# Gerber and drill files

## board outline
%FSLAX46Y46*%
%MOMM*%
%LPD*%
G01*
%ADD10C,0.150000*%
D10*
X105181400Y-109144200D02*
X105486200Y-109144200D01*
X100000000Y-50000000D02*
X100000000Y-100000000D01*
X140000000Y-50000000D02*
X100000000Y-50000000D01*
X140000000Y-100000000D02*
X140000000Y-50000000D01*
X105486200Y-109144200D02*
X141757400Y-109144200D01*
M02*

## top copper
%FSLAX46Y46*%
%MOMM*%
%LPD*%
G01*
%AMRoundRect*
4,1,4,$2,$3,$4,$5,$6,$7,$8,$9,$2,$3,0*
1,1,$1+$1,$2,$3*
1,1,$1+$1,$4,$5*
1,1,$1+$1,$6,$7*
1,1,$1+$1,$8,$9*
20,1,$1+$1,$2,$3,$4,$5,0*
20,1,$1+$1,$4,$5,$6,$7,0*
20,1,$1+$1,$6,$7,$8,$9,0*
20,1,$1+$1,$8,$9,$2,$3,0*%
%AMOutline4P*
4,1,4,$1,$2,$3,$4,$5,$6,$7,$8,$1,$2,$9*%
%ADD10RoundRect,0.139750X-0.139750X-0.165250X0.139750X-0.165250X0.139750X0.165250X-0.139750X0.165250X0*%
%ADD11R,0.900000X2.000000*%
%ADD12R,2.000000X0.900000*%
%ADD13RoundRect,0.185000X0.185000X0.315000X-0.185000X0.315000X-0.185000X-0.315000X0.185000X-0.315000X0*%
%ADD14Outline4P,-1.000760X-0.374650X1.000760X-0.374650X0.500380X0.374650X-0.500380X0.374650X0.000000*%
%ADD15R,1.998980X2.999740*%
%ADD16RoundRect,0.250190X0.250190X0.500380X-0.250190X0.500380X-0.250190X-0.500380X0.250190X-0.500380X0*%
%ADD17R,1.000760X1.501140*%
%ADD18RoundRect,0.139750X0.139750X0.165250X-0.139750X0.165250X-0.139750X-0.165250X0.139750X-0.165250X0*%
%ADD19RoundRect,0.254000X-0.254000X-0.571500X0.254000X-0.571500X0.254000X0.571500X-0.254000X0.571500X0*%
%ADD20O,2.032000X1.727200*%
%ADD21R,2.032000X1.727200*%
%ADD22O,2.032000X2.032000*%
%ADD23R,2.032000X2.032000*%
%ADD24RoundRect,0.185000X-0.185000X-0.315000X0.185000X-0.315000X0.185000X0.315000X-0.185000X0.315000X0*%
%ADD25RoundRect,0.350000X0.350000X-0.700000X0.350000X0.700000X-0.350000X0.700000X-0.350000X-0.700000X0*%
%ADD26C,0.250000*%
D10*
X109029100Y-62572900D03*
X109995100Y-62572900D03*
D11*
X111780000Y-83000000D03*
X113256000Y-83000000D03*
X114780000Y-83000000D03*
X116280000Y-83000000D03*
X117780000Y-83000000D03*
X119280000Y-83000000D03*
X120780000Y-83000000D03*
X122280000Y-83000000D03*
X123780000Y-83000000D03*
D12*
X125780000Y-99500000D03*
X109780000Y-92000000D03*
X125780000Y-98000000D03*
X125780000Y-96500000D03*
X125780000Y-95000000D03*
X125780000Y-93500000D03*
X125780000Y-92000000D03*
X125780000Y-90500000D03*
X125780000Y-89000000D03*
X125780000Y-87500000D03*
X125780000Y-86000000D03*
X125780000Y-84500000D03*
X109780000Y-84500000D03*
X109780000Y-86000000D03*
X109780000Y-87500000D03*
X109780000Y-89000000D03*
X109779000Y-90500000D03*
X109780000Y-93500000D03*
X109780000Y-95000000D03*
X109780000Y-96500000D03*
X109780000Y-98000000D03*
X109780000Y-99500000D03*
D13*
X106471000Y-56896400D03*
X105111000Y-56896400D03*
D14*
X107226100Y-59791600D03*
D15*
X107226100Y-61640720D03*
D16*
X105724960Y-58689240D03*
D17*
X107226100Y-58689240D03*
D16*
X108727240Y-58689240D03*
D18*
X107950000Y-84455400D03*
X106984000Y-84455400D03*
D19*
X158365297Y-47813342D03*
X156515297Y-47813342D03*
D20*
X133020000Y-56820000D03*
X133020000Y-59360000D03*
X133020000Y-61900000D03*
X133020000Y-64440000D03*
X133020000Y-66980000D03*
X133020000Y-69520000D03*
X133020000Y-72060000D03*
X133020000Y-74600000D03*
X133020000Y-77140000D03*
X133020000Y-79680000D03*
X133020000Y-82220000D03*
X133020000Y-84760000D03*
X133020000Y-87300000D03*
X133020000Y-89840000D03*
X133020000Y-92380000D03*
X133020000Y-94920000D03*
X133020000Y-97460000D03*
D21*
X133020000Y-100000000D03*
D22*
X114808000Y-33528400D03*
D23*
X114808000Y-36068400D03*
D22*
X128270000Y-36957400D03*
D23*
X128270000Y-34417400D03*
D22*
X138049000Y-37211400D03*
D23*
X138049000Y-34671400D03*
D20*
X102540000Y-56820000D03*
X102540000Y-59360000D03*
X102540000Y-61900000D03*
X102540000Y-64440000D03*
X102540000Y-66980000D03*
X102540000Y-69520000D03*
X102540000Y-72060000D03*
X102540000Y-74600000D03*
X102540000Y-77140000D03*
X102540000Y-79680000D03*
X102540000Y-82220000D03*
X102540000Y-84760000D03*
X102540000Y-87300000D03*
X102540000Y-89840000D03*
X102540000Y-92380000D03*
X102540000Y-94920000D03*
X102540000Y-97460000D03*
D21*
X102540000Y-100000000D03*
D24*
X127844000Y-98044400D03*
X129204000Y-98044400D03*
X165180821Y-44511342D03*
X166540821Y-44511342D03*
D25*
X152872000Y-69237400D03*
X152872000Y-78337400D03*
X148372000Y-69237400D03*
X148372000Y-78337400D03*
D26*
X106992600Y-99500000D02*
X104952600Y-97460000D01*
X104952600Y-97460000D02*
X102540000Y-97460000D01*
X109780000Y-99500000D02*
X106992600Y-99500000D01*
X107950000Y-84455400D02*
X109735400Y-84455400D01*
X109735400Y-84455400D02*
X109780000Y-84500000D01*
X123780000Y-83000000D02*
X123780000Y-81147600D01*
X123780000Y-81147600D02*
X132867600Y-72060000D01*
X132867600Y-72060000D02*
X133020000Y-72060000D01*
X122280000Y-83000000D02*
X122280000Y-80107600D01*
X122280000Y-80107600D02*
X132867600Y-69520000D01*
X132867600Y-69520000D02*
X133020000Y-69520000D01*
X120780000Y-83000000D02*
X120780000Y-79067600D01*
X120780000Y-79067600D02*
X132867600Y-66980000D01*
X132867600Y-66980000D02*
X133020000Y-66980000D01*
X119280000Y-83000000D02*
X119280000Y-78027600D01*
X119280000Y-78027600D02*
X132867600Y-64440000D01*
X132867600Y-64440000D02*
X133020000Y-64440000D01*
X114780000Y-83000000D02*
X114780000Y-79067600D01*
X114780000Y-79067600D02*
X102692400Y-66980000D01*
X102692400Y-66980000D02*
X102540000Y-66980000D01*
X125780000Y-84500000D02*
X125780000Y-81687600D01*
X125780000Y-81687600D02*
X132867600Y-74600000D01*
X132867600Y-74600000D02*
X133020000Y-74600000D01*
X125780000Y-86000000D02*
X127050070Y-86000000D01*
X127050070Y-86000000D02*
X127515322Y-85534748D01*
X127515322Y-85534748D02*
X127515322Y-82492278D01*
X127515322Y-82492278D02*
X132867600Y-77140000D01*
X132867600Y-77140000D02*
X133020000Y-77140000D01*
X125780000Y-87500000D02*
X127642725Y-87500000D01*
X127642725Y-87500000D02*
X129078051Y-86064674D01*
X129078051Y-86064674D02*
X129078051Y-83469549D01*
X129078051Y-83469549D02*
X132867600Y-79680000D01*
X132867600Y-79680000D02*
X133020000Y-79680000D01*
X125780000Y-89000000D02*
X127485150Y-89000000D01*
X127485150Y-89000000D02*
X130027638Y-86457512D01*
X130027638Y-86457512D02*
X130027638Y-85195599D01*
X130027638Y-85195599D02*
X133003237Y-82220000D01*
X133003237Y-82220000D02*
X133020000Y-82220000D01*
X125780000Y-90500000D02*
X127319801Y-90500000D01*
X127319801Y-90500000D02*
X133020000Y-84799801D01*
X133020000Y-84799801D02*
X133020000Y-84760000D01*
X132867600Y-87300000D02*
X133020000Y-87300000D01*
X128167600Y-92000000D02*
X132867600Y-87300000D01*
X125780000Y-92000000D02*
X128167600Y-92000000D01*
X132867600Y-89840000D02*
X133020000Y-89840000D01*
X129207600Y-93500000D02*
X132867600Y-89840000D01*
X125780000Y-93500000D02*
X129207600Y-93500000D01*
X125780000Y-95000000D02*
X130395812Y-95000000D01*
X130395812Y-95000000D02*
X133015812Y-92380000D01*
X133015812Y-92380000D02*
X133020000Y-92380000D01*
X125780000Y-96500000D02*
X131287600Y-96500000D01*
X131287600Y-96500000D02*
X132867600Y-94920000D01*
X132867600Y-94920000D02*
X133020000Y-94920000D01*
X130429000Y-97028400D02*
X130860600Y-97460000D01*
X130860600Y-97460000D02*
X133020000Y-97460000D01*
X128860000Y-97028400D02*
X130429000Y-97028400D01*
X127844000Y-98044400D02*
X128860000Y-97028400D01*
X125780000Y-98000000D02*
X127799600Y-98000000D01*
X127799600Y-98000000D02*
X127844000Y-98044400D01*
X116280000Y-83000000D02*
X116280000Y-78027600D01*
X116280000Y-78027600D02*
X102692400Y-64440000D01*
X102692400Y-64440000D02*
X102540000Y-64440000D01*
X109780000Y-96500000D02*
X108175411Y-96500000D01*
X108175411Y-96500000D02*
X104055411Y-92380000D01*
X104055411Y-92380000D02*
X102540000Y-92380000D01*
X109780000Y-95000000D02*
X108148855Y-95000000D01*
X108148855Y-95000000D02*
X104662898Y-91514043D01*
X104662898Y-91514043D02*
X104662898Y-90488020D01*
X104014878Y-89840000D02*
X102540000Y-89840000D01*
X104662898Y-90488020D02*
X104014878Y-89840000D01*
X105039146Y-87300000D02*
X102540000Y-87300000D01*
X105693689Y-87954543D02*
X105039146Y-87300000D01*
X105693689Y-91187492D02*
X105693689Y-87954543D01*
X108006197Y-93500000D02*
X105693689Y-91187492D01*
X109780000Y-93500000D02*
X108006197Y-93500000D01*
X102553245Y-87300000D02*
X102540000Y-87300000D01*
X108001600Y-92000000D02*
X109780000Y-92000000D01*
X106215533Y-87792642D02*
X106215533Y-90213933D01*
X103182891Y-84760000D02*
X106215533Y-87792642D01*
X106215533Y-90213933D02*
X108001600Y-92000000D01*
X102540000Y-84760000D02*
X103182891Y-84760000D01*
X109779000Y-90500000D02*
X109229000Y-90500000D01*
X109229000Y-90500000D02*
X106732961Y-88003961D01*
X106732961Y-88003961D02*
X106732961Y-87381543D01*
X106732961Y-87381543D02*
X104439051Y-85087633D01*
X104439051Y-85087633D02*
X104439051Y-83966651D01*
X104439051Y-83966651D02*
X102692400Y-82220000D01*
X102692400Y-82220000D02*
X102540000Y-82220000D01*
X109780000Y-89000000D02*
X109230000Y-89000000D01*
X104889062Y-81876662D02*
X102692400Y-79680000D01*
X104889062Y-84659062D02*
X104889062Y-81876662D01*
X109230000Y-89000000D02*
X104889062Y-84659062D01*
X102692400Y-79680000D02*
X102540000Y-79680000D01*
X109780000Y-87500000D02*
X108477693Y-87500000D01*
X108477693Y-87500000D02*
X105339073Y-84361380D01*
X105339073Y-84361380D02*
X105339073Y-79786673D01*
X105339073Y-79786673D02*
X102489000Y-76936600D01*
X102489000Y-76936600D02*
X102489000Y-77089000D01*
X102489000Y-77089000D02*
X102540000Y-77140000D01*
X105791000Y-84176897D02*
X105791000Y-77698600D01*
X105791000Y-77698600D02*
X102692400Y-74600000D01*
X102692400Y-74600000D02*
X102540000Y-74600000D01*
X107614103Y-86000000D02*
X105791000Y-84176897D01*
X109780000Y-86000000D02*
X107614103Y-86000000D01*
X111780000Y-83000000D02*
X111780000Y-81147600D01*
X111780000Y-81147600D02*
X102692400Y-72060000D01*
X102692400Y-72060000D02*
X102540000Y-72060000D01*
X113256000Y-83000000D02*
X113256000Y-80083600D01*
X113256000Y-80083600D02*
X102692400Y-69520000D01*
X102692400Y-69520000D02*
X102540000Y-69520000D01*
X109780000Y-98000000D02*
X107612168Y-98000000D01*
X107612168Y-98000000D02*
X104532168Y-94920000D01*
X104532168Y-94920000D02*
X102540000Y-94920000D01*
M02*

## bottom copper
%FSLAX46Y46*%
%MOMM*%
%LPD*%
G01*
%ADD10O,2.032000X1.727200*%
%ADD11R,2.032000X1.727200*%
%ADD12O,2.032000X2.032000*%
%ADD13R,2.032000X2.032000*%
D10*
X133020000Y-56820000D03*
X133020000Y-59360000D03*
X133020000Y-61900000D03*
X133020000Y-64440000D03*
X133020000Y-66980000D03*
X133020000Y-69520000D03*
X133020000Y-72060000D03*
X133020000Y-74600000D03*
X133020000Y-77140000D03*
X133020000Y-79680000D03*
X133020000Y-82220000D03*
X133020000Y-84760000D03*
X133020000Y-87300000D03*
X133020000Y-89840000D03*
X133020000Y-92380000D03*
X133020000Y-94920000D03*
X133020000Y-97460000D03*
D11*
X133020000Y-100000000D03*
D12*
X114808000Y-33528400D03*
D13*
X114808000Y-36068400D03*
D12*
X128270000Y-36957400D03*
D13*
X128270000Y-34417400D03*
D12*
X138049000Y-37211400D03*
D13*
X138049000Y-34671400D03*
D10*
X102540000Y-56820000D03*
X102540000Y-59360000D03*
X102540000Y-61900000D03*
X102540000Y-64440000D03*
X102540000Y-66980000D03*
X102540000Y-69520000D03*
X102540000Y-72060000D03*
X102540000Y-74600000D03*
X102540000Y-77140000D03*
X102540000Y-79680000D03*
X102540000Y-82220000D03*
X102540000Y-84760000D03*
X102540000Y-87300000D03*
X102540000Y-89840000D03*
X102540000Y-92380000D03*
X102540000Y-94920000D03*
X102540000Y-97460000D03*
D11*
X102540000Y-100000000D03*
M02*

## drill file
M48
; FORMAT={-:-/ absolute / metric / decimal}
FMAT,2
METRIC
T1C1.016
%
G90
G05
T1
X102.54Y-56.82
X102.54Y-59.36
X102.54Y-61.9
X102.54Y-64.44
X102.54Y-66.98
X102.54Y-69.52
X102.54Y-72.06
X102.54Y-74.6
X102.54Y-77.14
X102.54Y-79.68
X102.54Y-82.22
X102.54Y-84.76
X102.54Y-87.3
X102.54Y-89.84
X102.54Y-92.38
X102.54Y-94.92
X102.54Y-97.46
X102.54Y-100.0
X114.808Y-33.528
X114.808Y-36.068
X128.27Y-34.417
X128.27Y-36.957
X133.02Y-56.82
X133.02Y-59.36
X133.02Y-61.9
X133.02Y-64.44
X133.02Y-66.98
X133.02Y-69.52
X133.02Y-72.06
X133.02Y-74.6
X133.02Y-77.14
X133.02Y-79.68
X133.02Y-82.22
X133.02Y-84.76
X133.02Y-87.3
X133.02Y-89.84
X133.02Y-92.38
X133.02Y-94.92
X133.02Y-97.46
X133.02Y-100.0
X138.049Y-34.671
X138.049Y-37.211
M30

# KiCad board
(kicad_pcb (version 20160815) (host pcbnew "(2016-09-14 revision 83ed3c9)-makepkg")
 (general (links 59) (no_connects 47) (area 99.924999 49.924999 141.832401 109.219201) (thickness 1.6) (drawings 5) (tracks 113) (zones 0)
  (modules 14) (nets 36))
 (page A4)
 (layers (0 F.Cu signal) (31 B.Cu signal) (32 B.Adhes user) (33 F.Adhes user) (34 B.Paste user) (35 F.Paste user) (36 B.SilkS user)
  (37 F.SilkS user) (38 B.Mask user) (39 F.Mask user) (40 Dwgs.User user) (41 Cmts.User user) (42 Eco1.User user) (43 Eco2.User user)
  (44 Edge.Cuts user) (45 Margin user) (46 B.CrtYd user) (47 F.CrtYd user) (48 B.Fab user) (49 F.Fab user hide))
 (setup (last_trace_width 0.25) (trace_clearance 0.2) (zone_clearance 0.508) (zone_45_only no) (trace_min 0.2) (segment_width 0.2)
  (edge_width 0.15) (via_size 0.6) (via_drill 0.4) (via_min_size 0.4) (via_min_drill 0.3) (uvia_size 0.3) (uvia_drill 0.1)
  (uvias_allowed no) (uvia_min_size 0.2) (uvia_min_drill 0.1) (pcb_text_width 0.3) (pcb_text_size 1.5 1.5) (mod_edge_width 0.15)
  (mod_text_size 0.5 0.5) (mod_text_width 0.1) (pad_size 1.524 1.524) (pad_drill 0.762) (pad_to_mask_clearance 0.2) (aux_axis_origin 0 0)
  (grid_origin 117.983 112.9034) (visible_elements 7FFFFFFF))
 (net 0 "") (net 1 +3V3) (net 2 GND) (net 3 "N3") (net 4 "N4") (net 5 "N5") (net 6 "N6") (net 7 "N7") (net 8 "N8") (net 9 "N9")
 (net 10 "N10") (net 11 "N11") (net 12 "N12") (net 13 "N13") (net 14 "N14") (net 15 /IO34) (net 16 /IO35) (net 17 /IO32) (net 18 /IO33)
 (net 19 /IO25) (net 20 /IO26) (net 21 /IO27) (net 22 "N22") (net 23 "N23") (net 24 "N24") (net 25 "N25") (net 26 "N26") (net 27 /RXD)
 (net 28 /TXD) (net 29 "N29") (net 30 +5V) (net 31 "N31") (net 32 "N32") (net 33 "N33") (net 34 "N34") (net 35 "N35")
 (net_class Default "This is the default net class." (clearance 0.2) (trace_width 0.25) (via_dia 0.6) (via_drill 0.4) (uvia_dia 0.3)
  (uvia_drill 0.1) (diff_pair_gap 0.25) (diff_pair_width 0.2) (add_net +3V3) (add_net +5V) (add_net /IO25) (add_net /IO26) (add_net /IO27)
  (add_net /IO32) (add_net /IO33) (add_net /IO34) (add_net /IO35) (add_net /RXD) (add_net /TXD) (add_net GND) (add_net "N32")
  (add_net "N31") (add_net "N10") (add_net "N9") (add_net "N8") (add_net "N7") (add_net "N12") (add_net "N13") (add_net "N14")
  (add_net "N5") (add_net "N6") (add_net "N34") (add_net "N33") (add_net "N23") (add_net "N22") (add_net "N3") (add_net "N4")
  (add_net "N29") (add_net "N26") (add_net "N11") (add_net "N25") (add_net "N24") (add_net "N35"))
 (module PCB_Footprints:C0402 (layer F.Cu) (at 109.5121 62.5729)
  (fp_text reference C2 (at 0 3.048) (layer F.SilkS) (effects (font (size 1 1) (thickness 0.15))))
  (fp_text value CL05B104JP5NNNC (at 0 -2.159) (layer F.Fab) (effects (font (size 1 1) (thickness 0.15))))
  (pad 1 smd roundrect (at -0.483 0) (size 0.559 0.61) (layers F.Cu F.Paste F.Mask) (roundrect_rratio 0.25) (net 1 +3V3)
   (solder_mask_margin 0.102))
  (pad 2 smd roundrect (at 0.483 0) (size 0.559 0.61) (layers F.Cu F.Paste F.Mask) (roundrect_rratio 0.25) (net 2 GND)
   (solder_mask_margin 0.102)))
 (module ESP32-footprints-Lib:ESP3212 (layer F.Cu) (at 117.78 95 180)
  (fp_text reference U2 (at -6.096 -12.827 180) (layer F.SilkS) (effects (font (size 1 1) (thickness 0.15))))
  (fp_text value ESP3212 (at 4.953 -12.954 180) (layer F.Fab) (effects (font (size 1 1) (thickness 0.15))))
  (pad 20 smd rect (at 6 12 180) (size 0.9 2) (layers F.Cu F.Paste F.Mask) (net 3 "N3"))
  (pad 19 smd rect (at 4.524 12 180) (size 0.9 2) (layers F.Cu F.Paste F.Mask) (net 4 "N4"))
  (pad 18 smd rect (at 3 12 180) (size 0.9 2) (layers F.Cu F.Paste F.Mask) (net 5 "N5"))
  (pad 17 smd rect (at 1.5 12 180) (size 0.9 2) (layers F.Cu F.Paste F.Mask) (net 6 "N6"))
  (pad 16 smd rect (at 0 12 180) (size 0.9 2) (layers F.Cu F.Paste F.Mask) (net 2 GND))
  (pad 15 smd rect (at -1.5 12 180) (size 0.9 2) (layers F.Cu F.Paste F.Mask) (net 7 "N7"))
  (pad 14 smd rect (at -3 12 180) (size 0.9 2) (layers F.Cu F.Paste F.Mask) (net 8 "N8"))
  (pad 13 smd rect (at -4.5 12 180) (size 0.9 2) (layers F.Cu F.Paste F.Mask) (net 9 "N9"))
  (pad 12 smd rect (at -6 12 180) (size 0.9 2) (layers F.Cu F.Paste F.Mask) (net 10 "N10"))
  (pad 1 smd rect (at -8 -4.5 180) (size 2 0.9) (layers F.Cu F.Paste F.Mask) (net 2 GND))
  (pad 26 smd rect (at 8 3 180) (size 2 0.9) (layers F.Cu F.Paste F.Mask) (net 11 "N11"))
  (pad 2 smd rect (at -8 -3 180) (size 2 0.9) (layers F.Cu F.Paste F.Mask) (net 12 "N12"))
  (pad 3 smd rect (at -8 -1.5 180) (size 2 0.9) (layers F.Cu F.Paste F.Mask) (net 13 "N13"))
  (pad 4 smd rect (at -8 0 180) (size 2 0.9) (layers F.Cu F.Paste F.Mask) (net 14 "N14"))
  (pad 5 smd rect (at -8 1.5 180) (size 2 0.9) (layers F.Cu F.Paste F.Mask) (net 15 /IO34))
  (pad 6 smd rect (at -8 3 180) (size 2 0.9) (layers F.Cu F.Paste F.Mask) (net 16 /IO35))
  (pad 7 smd rect (at -8 4.5 180) (size 2 0.9) (layers F.Cu F.Paste F.Mask) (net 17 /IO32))
  (pad 8 smd rect (at -8 6 180) (size 2 0.9) (layers F.Cu F.Paste F.Mask) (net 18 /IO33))
  (pad 9 smd rect (at -8 7.5 180) (size 2 0.9) (layers F.Cu F.Paste F.Mask) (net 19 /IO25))
  (pad 10 smd rect (at -8 9 180) (size 2 0.9) (layers F.Cu F.Paste F.Mask) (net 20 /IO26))
  (pad 11 smd rect (at -8 10.5 180) (size 2 0.9) (layers F.Cu F.Paste F.Mask) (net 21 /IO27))
  (pad 21 smd rect (at 8 10.5 180) (size 2 0.9) (layers F.Cu F.Paste F.Mask) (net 1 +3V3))
  (pad 22 smd rect (at 8 9 180) (size 2 0.9) (layers F.Cu F.Paste F.Mask) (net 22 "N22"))
  (pad 23 smd rect (at 8 7.5 180) (size 2 0.9) (layers F.Cu F.Paste F.Mask) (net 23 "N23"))
  (pad 24 smd rect (at 8 6 180) (size 2 0.9) (layers F.Cu F.Paste F.Mask) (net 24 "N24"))
  (pad 25 smd rect (at 8.001 4.5 180) (size 2 0.9) (layers F.Cu F.Paste F.Mask) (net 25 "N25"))
  (pad 27 smd rect (at 8 1.5 180) (size 2 0.9) (layers F.Cu F.Paste F.Mask) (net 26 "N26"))
  (pad 28 smd rect (at 8 0 180) (size 2 0.9) (layers F.Cu F.Paste F.Mask) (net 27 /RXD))
  (pad 29 smd rect (at 8 -1.5 180) (size 2 0.9) (layers F.Cu F.Paste F.Mask) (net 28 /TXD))
  (pad 30 smd rect (at 8 -3 180) (size 2 0.9) (layers F.Cu F.Paste F.Mask) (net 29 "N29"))
  (pad 31 smd rect (at 8 -4.5 180) (size 2 0.9) (layers F.Cu F.Paste F.Mask) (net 2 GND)))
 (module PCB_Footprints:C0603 (layer F.Cu) (at 105.791 56.8964 180)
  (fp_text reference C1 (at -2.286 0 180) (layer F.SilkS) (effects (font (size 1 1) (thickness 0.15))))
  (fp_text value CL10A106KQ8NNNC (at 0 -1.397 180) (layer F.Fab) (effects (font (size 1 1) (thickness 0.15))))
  (pad 1 smd roundrect (at -0.68 0 180) (size 0.74 1) (layers F.Cu F.Paste F.Mask) (roundrect_rratio 0.25) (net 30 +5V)
   (solder_mask_margin 0.102))
  (pad 2 smd roundrect (at 0.68 0 180) (size 0.74 1) (layers F.Cu F.Paste F.Mask) (roundrect_rratio 0.25) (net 2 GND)
   (solder_mask_margin 0.102)))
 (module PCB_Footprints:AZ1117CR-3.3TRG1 (layer F.Cu) (at 107.2261 60.5409 180)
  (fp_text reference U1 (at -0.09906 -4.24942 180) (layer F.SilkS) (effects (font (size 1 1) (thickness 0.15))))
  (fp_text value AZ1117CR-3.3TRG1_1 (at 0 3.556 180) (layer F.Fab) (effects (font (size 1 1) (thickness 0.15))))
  (pad 2 smd trapezoid (at 0 0.7493) (size 1.50114 0.7493) (rect_delta 0 0.50038) (layers F.Cu F.Paste F.Mask) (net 1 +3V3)
   (solder_mask_margin 0.102))
  (pad 2 smd rect (at 0 -1.09982 180) (size 1.99898 2.99974) (layers F.Cu F.Paste F.Mask) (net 1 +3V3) (solder_mask_margin 0.102))
  (pad 3 smd roundrect (at 1.50114 1.85166 180) (size 1.00076 1.50114) (layers F.Cu F.Paste F.Mask) (roundrect_rratio 0.25) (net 30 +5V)
   (solder_mask_margin 0.102))
  (pad 2 smd rect (at 0 1.85166 180) (size 1.00076 1.50114) (layers F.Cu F.Paste F.Mask) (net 1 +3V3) (solder_mask_margin 0.102))
  (pad 1 smd roundrect (at -1.50114 1.85166 180) (size 1.00076 1.50114) (layers F.Cu F.Paste F.Mask) (roundrect_rratio 0.25) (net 2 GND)
   (solder_mask_margin 0.102)))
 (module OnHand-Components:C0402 (layer F.Cu) (at 107.467 84.4554 180)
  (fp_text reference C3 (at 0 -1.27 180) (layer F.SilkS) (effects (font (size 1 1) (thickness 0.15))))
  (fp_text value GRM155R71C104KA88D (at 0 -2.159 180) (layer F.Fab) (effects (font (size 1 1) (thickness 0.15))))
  (pad 1 smd roundrect (at -0.483 0 180) (size 0.559 0.61) (layers F.Cu F.Paste F.Mask) (roundrect_rratio 0.25) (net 1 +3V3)
   (solder_mask_margin 0.102))
  (pad 2 smd roundrect (at 0.483 0 180) (size 0.559 0.61) (layers F.Cu F.Paste F.Mask) (roundrect_rratio 0.25) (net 2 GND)
   (solder_mask_margin 0.102)))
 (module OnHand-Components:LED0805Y (layer F.Cu) (at 157.440297 47.813342)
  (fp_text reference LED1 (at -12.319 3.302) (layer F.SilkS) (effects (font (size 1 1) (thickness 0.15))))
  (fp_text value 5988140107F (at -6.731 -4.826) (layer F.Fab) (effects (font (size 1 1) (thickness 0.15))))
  (pad 2 smd roundrect (at 0.925 0) (size 1.016 1.651) (layers F.Cu F.Paste F.Mask) (roundrect_rratio 0.25) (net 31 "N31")
   (solder_mask_margin 0.102))
  (pad 1 smd roundrect (at -0.925 0) (size 1.016 1.651) (layers F.Cu F.Paste F.Mask) (roundrect_rratio 0.25) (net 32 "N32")
   (solder_mask_margin 0.102)))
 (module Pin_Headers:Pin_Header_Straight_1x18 (layer F.Cu) (at 133.02 100 180)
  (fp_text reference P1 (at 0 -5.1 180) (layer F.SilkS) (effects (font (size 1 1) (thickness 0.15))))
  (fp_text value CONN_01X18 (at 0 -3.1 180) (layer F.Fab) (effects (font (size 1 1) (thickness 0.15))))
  (pad 18 thru_hole oval (at 0 43.18 180) (size 2.032 1.7272) (drill 1.016) (layers *.Cu *.Mask F.SilkS) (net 2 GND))
  (pad 17 thru_hole oval (at 0 40.64 180) (size 2.032 1.7272) (drill 1.016) (layers *.Cu *.Mask F.SilkS) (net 30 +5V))
  (pad 16 thru_hole oval (at 0 38.1 180) (size 2.032 1.7272) (drill 1.016) (layers *.Cu *.Mask F.SilkS) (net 1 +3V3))
  (pad 15 thru_hole oval (at 0 35.56 180) (size 2.032 1.7272) (drill 1.016) (layers *.Cu *.Mask F.SilkS) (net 7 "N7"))
  (pad 14 thru_hole oval (at 0 33.02 180) (size 2.032 1.7272) (drill 1.016) (layers *.Cu *.Mask F.SilkS) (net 8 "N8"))
  (pad 13 thru_hole oval (at 0 30.48 180) (size 2.032 1.7272) (drill 1.016) (layers *.Cu *.Mask F.SilkS) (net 9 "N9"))
  (pad 12 thru_hole oval (at 0 27.94 180) (size 2.032 1.7272) (drill 1.016) (layers *.Cu *.Mask F.SilkS) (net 10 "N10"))
  (pad 11 thru_hole oval (at 0 25.4 180) (size 2.032 1.7272) (drill 1.016) (layers *.Cu *.Mask F.SilkS) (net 21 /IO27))
  (pad 10 thru_hole oval (at 0 22.86 180) (size 2.032 1.7272) (drill 1.016) (layers *.Cu *.Mask F.SilkS) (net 20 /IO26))
  (pad 9 thru_hole oval (at 0 20.32 180) (size 2.032 1.7272) (drill 1.016) (layers *.Cu *.Mask F.SilkS) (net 19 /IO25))
  (pad 8 thru_hole oval (at 0 17.78 180) (size 2.032 1.7272) (drill 1.016) (layers *.Cu *.Mask F.SilkS) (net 18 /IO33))
  (pad 7 thru_hole oval (at 0 15.24 180) (size 2.032 1.7272) (drill 1.016) (layers *.Cu *.Mask F.SilkS) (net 17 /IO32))
  (pad 6 thru_hole oval (at 0 12.7 180) (size 2.032 1.7272) (drill 1.016) (layers *.Cu *.Mask F.SilkS) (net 16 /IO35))
  (pad 5 thru_hole oval (at 0 10.16 180) (size 2.032 1.7272) (drill 1.016) (layers *.Cu *.Mask F.SilkS) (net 15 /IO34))
  (pad 4 thru_hole oval (at 0 7.62 180) (size 2.032 1.7272) (drill 1.016) (layers *.Cu *.Mask F.SilkS) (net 14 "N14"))
  (pad 3 thru_hole oval (at 0 5.08 180) (size 2.032 1.7272) (drill 1.016) (layers *.Cu *.Mask F.SilkS) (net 13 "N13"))
  (pad 2 thru_hole oval (at 0 2.54 180) (size 2.032 1.7272) (drill 1.016) (layers *.Cu *.Mask F.SilkS) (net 12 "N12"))
  (pad 1 thru_hole rect (at 0 0 180) (size 2.032 1.7272) (drill 1.016) (layers *.Cu *.Mask F.SilkS) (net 2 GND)))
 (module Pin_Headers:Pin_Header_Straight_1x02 (layer F.Cu) (at 114.808 36.0684 180)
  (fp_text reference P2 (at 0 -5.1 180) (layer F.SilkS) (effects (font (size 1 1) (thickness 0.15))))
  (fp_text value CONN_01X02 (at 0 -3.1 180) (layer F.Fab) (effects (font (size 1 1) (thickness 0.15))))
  (pad 2 thru_hole oval (at 0 2.54 180) (size 2.032 2.032) (drill 1.016) (layers *.Cu *.Mask F.SilkS) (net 2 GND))
  (pad 1 thru_hole rect (at 0 0 180) (size 2.032 2.032) (drill 1.016) (layers *.Cu *.Mask F.SilkS) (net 5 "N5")))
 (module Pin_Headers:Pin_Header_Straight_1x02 (layer F.Cu) (at 128.27 34.4174)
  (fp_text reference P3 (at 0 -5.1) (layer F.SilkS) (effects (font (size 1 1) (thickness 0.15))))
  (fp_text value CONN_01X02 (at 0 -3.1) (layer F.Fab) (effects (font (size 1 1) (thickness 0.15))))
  (pad 2 thru_hole oval (at 0 2.54) (size 2.032 2.032) (drill 1.016) (layers *.Cu *.Mask F.SilkS) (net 2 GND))
  (pad 1 thru_hole rect (at 0 0) (size 2.032 2.032) (drill 1.016) (layers *.Cu *.Mask F.SilkS) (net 6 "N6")))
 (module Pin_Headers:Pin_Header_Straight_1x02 (layer F.Cu) (at 138.049 34.6714)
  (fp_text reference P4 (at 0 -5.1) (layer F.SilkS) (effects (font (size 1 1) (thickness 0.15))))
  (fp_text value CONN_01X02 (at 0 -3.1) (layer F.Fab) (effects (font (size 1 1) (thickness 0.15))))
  (pad 2 thru_hole oval (at 0 2.54) (size 2.032 2.032) (drill 1.016) (layers *.Cu *.Mask F.SilkS) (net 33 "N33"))
  (pad 1 thru_hole rect (at 0 0) (size 2.032 2.032) (drill 1.016) (layers *.Cu *.Mask F.SilkS) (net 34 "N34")))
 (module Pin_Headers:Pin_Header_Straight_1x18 (layer F.Cu) (at 102.54 100 180)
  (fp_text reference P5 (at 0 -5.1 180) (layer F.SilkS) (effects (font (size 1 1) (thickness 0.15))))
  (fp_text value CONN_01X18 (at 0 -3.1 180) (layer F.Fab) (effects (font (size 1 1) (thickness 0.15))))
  (pad 18 thru_hole oval (at 0 43.18 180) (size 2.032 1.7272) (drill 1.016) (layers *.Cu *.Mask F.SilkS) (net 2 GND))
  (pad 17 thru_hole oval (at 0 40.64 180) (size 2.032 1.7272) (drill 1.016) (layers *.Cu *.Mask F.SilkS) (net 30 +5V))
  (pad 16 thru_hole oval (at 0 38.1 180) (size 2.032 1.7272) (drill 1.016) (layers *.Cu *.Mask F.SilkS) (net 1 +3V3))
  (pad 15 thru_hole oval (at 0 35.56 180) (size 2.032 1.7272) (drill 1.016) (layers *.Cu *.Mask F.SilkS) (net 6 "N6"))
  (pad 14 thru_hole oval (at 0 33.02 180) (size 2.032 1.7272) (drill 1.016) (layers *.Cu *.Mask F.SilkS) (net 5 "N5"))
  (pad 13 thru_hole oval (at 0 30.48 180) (size 2.032 1.7272) (drill 1.016) (layers *.Cu *.Mask F.SilkS) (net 4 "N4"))
  (pad 12 thru_hole oval (at 0 27.94 180) (size 2.032 1.7272) (drill 1.016) (layers *.Cu *.Mask F.SilkS) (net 3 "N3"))
  (pad 11 thru_hole oval (at 0 25.4 180) (size 2.032 1.7272) (drill 1.016) (layers *.Cu *.Mask F.SilkS) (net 22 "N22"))
  (pad 10 thru_hole oval (at 0 22.86 180) (size 2.032 1.7272) (drill 1.016) (layers *.Cu *.Mask F.SilkS) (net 23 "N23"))
  (pad 9 thru_hole oval (at 0 20.32 180) (size 2.032 1.7272) (drill 1.016) (layers *.Cu *.Mask F.SilkS) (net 24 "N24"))
  (pad 8 thru_hole oval (at 0 17.78 180) (size 2.032 1.7272) (drill 1.016) (layers *.Cu *.Mask F.SilkS) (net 25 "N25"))
  (pad 7 thru_hole oval (at 0 15.24 180) (size 2.032 1.7272) (drill 1.016) (layers *.Cu *.Mask F.SilkS) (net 11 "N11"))
  (pad 6 thru_hole oval (at 0 12.7 180) (size 2.032 1.7272) (drill 1.016) (layers *.Cu *.Mask F.SilkS) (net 26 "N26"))
  (pad 5 thru_hole oval (at 0 10.16 180) (size 2.032 1.7272) (drill 1.016) (layers *.Cu *.Mask F.SilkS) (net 27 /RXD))
  (pad 4 thru_hole oval (at 0 7.62 180) (size 2.032 1.7272) (drill 1.016) (layers *.Cu *.Mask F.SilkS) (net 28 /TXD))
  (pad 3 thru_hole oval (at 0 5.08 180) (size 2.032 1.7272) (drill 1.016) (layers *.Cu *.Mask F.SilkS) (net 29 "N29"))
  (pad 2 thru_hole oval (at 0 2.54 180) (size 2.032 1.7272) (drill 1.016) (layers *.Cu *.Mask F.SilkS) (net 2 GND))
  (pad 1 thru_hole rect (at 0 0 180) (size 2.032 1.7272) (drill 1.016) (layers *.Cu *.Mask F.SilkS) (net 2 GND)))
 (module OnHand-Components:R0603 (layer F.Cu) (at 128.524 98.0444)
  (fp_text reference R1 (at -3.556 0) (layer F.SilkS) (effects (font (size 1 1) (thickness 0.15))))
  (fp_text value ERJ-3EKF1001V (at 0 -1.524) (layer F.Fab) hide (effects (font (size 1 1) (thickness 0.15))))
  (pad 1 smd roundrect (at -0.68 0) (size 0.74 1) (layers F.Cu F.Paste F.Mask) (roundrect_rratio 0.25) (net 12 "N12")
   (solder_mask_margin 0.102))
  (pad 2 smd roundrect (at 0.68 0) (size 0.74 1) (layers F.Cu F.Paste F.Mask) (roundrect_rratio 0.25) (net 1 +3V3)
   (solder_mask_margin 0.102)))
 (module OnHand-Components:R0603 (layer F.Cu) (at 165.860821 44.511342)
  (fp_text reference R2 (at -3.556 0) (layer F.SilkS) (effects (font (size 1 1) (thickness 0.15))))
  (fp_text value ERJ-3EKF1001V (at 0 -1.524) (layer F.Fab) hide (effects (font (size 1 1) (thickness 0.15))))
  (pad 1 smd roundrect (at -0.68 0) (size 0.74 1) (layers F.Cu F.Paste F.Mask) (roundrect_rratio 0.25) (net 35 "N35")
   (solder_mask_margin 0.102))
  (pad 2 smd roundrect (at 0.68 0) (size 0.74 1) (layers F.Cu F.Paste F.Mask) (roundrect_rratio 0.25) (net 34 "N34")
   (solder_mask_margin 0.102)))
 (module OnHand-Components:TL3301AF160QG (layer F.Cu) (at 150.622 73.7874 90)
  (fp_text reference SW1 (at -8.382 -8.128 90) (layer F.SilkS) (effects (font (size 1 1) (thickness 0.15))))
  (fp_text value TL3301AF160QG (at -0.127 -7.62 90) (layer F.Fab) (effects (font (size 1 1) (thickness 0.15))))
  (pad 2 smd roundrect (at 4.55 2.25 90) (size 2.1 1.4) (layers F.Cu F.Paste F.Mask) (roundrect_rratio 0.25) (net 12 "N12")
   (solder_mask_margin 0.102))
  (pad 2 smd roundrect (at -4.55 2.25 90) (size 2.1 1.4) (layers F.Cu F.Paste F.Mask) (roundrect_rratio 0.25) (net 12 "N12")
   (solder_mask_margin 0.102))
  (pad 1 smd roundrect (at 4.55 -2.25 90) (size 2.1 1.4) (layers F.Cu F.Paste F.Mask) (roundrect_rratio 0.25) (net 2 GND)
   (solder_mask_margin 0.102))
  (pad 1 smd roundrect (at -4.55 -2.25 90) (size 2.1 1.4) (layers F.Cu F.Paste F.Mask) (roundrect_rratio 0.25) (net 2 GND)
   (solder_mask_margin 0.102)))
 (gr_line (start 105.1814 109.1442) (end 105.4862 109.1442) (angle 90) (layer Edge.Cuts) (width 0.15))
 (gr_line (start 100 50) (end 100 100) (angle 90) (layer Edge.Cuts) (width 0.15))
 (gr_line (start 140 50) (end 100 50) (angle 90) (layer Edge.Cuts) (width 0.15))
 (gr_line (start 140 100) (end 140 50) (angle 90) (layer Edge.Cuts) (width 0.15))
 (gr_line (start 105.4862 109.1442) (end 141.7574 109.1442) (angle 90) (layer Edge.Cuts) (width 0.15))
 (segment (start 106.9926 99.5) (end 104.9526 97.46) (width 0.25) (layer F.Cu) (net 2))
 (segment (start 104.9526 97.46) (end 102.54 97.46) (width 0.25) (layer F.Cu) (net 2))
 (segment (start 109.78 99.5) (end 106.9926 99.5) (width 0.25) (layer F.Cu) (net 2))
 (segment (start 107.95 84.4554) (end 109.7354 84.4554) (width 0.25) (layer F.Cu) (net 1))
 (segment (start 109.7354 84.4554) (end 109.78 84.5) (width 0.25) (layer F.Cu) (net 1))
 (segment (start 123.78 83) (end 123.78 81.1476) (width 0.25) (layer F.Cu) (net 10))
 (segment (start 123.78 81.1476) (end 132.8676 72.06) (width 0.25) (layer F.Cu) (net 10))
 (segment (start 132.8676 72.06) (end 133.02 72.06) (width 0.25) (layer F.Cu) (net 10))
 (segment (start 122.28 83) (end 122.28 80.1076) (width 0.25) (layer F.Cu) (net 9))
 (segment (start 122.28 80.1076) (end 132.8676 69.52) (width 0.25) (layer F.Cu) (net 9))
 (segment (start 132.8676 69.52) (end 133.02 69.52) (width 0.25) (layer F.Cu) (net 9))
 (segment (start 120.78 83) (end 120.78 79.0676) (width 0.25) (layer F.Cu) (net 8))
 (segment (start 120.78 79.0676) (end 132.8676 66.98) (width 0.25) (layer F.Cu) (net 8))
 (segment (start 132.8676 66.98) (end 133.02 66.98) (width 0.25) (layer F.Cu) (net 8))
 (segment (start 119.28 83) (end 119.28 78.0276) (width 0.25) (layer F.Cu) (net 7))
 (segment (start 119.28 78.0276) (end 132.8676 64.44) (width 0.25) (layer F.Cu) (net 7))
 (segment (start 132.8676 64.44) (end 133.02 64.44) (width 0.25) (layer F.Cu) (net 7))
 (segment (start 114.78 83) (end 114.78 79.0676) (width 0.25) (layer F.Cu) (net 5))
 (segment (start 114.78 79.0676) (end 102.6924 66.98) (width 0.25) (layer F.Cu) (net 5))
 (segment (start 102.6924 66.98) (end 102.54 66.98) (width 0.25) (layer F.Cu) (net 5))
 (segment (start 125.78 84.5) (end 125.78 81.6876) (width 0.25) (layer F.Cu) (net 21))
 (segment (start 125.78 81.6876) (end 132.8676 74.6) (width 0.25) (layer F.Cu) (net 21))
 (segment (start 132.8676 74.6) (end 133.02 74.6) (width 0.25) (layer F.Cu) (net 21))
 (segment (start 125.78 86) (end 127.05007 86) (width 0.25) (layer F.Cu) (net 20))
 (segment (start 127.05007 86) (end 127.515322 85.534748) (width 0.25) (layer F.Cu) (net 20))
 (segment (start 127.515322 85.534748) (end 127.515322 82.492278) (width 0.25) (layer F.Cu) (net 20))
 (segment (start 127.515322 82.492278) (end 132.8676 77.14) (width 0.25) (layer F.Cu) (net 20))
 (segment (start 132.8676 77.14) (end 133.02 77.14) (width 0.25) (layer F.Cu) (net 20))
 (segment (start 125.78 87.5) (end 127.642725 87.5) (width 0.25) (layer F.Cu) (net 19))
 (segment (start 127.642725 87.5) (end 129.078051 86.064674) (width 0.25) (layer F.Cu) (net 19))
 (segment (start 129.078051 86.064674) (end 129.078051 83.469549) (width 0.25) (layer F.Cu) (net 19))
 (segment (start 129.078051 83.469549) (end 132.8676 79.68) (width 0.25) (layer F.Cu) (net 19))
 (segment (start 132.8676 79.68) (end 133.02 79.68) (width 0.25) (layer F.Cu) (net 19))
 (segment (start 125.78 89) (end 127.48515 89) (width 0.25) (layer F.Cu) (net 18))
 (segment (start 127.48515 89) (end 130.027638 86.457512) (width 0.25) (layer F.Cu) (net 18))
 (segment (start 130.027638 86.457512) (end 130.027638 85.195599) (width 0.25) (layer F.Cu) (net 18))
 (segment (start 130.027638 85.195599) (end 133.003237 82.22) (width 0.25) (layer F.Cu) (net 18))
 (segment (start 133.003237 82.22) (end 133.02 82.22) (width 0.25) (layer F.Cu) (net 18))
 (segment (start 125.78 90.5) (end 127.319801 90.5) (width 0.25) (layer F.Cu) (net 17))
 (segment (start 127.319801 90.5) (end 133.02 84.799801) (width 0.25) (layer F.Cu) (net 17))
 (segment (start 133.02 84.799801) (end 133.02 84.76) (width 0.25) (layer F.Cu) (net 17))
 (segment (start 132.8676 87.3) (end 133.02 87.3) (width 0.25) (layer F.Cu) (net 16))
 (segment (start 128.1676 92) (end 132.8676 87.3) (width 0.25) (layer F.Cu) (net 16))
 (segment (start 125.78 92) (end 128.1676 92) (width 0.25) (layer F.Cu) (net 16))
 (segment (start 132.8676 89.84) (end 133.02 89.84) (width 0.25) (layer F.Cu) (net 15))
 (segment (start 129.2076 93.5) (end 132.8676 89.84) (width 0.25) (layer F.Cu) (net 15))
 (segment (start 125.78 93.5) (end 129.2076 93.5) (width 0.25) (layer F.Cu) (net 15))
 (segment (start 125.78 95) (end 130.395812 95) (width 0.25) (layer F.Cu) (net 14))
 (segment (start 130.395812 95) (end 133.015812 92.38) (width 0.25) (layer F.Cu) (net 14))
 (segment (start 133.015812 92.38) (end 133.02 92.38) (width 0.25) (layer F.Cu) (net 14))
 (segment (start 125.78 96.5) (end 131.2876 96.5) (width 0.25) (layer F.Cu) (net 13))
 (segment (start 131.2876 96.5) (end 132.8676 94.92) (width 0.25) (layer F.Cu) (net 13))
 (segment (start 132.8676 94.92) (end 133.02 94.92) (width 0.25) (layer F.Cu) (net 13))
 (segment (start 130.429 97.0284) (end 130.8606 97.46) (width 0.25) (layer F.Cu) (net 12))
 (segment (start 130.8606 97.46) (end 133.02 97.46) (width 0.25) (layer F.Cu) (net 12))
 (segment (start 128.86 97.0284) (end 130.429 97.0284) (width 0.25) (layer F.Cu) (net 12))
 (segment (start 127.844 98.0444) (end 128.86 97.0284) (width 0.25) (layer F.Cu) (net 12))
 (segment (start 125.78 98) (end 127.7996 98) (width 0.25) (layer F.Cu) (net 12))
 (segment (start 127.7996 98) (end 127.844 98.0444) (width 0.25) (layer F.Cu) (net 12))
 (segment (start 116.28 83) (end 116.28 78.0276) (width 0.25) (layer F.Cu) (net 6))
 (segment (start 116.28 78.0276) (end 102.6924 64.44) (width 0.25) (layer F.Cu) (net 6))
 (segment (start 102.6924 64.44) (end 102.54 64.44) (width 0.25) (layer F.Cu) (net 6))
 (segment (start 109.78 96.5) (end 108.175411 96.5) (width 0.25) (layer F.Cu) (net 28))
 (segment (start 108.175411 96.5) (end 104.055411 92.38) (width 0.25) (layer F.Cu) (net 28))
 (segment (start 104.055411 92.38) (end 102.54 92.38) (width 0.25) (layer F.Cu) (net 28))
 (segment (start 109.78 95) (end 108.148855 95) (width 0.25) (layer F.Cu) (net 27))
 (segment (start 108.148855 95) (end 104.662898 91.514043) (width 0.25) (layer F.Cu) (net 27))
 (segment (start 104.662898 91.514043) (end 104.662898 90.48802) (width 0.25) (layer F.Cu) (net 27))
 (segment (start 104.014878 89.84) (end 102.54 89.84) (width 0.25) (layer F.Cu) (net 27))
 (segment (start 104.662898 90.48802) (end 104.014878 89.84) (width 0.25) (layer F.Cu) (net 27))
 (segment (start 105.039146 87.3) (end 102.54 87.3) (width 0.25) (layer F.Cu) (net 26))
 (segment (start 105.693689 87.954543) (end 105.039146 87.3) (width 0.25) (layer F.Cu) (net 26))
 (segment (start 105.693689 91.187492) (end 105.693689 87.954543) (width 0.25) (layer F.Cu) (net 26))
 (segment (start 108.006197 93.5) (end 105.693689 91.187492) (width 0.25) (layer F.Cu) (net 26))
 (segment (start 109.78 93.5) (end 108.006197 93.5) (width 0.25) (layer F.Cu) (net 26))
 (segment (start 102.553245 87.3) (end 102.54 87.3) (width 0.25) (layer F.Cu) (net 26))
 (segment (start 108.0016 92) (end 109.78 92) (width 0.25) (layer F.Cu) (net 11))
 (segment (start 106.215533 87.792642) (end 106.215533 90.213933) (width 0.25) (layer F.Cu) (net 11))
 (segment (start 103.182891 84.76) (end 106.215533 87.792642) (width 0.25) (layer F.Cu) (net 11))
 (segment (start 106.215533 90.213933) (end 108.0016 92) (width 0.25) (layer F.Cu) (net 11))
 (segment (start 102.54 84.76) (end 103.182891 84.76) (width 0.25) (layer F.Cu) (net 11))
 (segment (start 109.779 90.5) (end 109.229 90.5) (width 0.25) (layer F.Cu) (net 25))
 (segment (start 109.229 90.5) (end 106.732961 88.003961) (width 0.25) (layer F.Cu) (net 25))
 (segment (start 106.732961 88.003961) (end 106.732961 87.381543) (width 0.25) (layer F.Cu) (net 25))
 (segment (start 106.732961 87.381543) (end 104.439051 85.087633) (width 0.25) (layer F.Cu) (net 25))
 (segment (start 104.439051 85.087633) (end 104.439051 83.966651) (width 0.25) (layer F.Cu) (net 25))
 (segment (start 104.439051 83.966651) (end 102.6924 82.22) (width 0.25) (layer F.Cu) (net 25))
 (segment (start 102.6924 82.22) (end 102.54 82.22) (width 0.25) (layer F.Cu) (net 25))
 (segment (start 109.78 89) (end 109.23 89) (width 0.25) (layer F.Cu) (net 24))
 (segment (start 104.889062 81.876662) (end 102.6924 79.68) (width 0.25) (layer F.Cu) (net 24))
 (segment (start 104.889062 84.659062) (end 104.889062 81.876662) (width 0.25) (layer F.Cu) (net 24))
 (segment (start 109.23 89) (end 104.889062 84.659062) (width 0.25) (layer F.Cu) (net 24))
 (segment (start 102.6924 79.68) (end 102.54 79.68) (width 0.25) (layer F.Cu) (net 24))
 (segment (start 109.78 87.5) (end 108.477693 87.5) (width 0.25) (layer F.Cu) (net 23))
 (segment (start 108.477693 87.5) (end 105.339073 84.36138) (width 0.25) (layer F.Cu) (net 23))
 (segment (start 105.339073 84.36138) (end 105.339073 79.786673) (width 0.25) (layer F.Cu) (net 23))
 (segment (start 105.339073 79.786673) (end 102.489 76.9366) (width 0.25) (layer F.Cu) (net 23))
 (segment (start 102.489 76.9366) (end 102.489 77.089) (width 0.25) (layer F.Cu) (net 23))
 (segment (start 102.489 77.089) (end 102.54 77.14) (width 0.25) (layer F.Cu) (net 23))
 (segment (start 105.791 84.176897) (end 105.791 77.6986) (width 0.25) (layer F.Cu) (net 22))
 (segment (start 105.791 77.6986) (end 102.6924 74.6) (width 0.25) (layer F.Cu) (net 22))
 (segment (start 102.6924 74.6) (end 102.54 74.6) (width 0.25) (layer F.Cu) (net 22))
 (segment (start 107.614103 86) (end 105.791 84.176897) (width 0.25) (layer F.Cu) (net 22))
 (segment (start 109.78 86) (end 107.614103 86) (width 0.25) (layer F.Cu) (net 22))
 (segment (start 111.78 83) (end 111.78 81.1476) (width 0.25) (layer F.Cu) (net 3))
 (segment (start 111.78 81.1476) (end 102.6924 72.06) (width 0.25) (layer F.Cu) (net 3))
 (segment (start 102.6924 72.06) (end 102.54 72.06) (width 0.25) (layer F.Cu) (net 3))
 (segment (start 113.256 83) (end 113.256 80.0836) (width 0.25) (layer F.Cu) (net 4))
 (segment (start 113.256 80.0836) (end 102.6924 69.52) (width 0.25) (layer F.Cu) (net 4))
 (segment (start 102.6924 69.52) (end 102.54 69.52) (width 0.25) (layer F.Cu) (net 4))
 (segment (start 109.78 98) (end 107.612168 98) (width 0.25) (layer F.Cu) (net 29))
 (segment (start 107.612168 98) (end 104.532168 94.92) (width 0.25) (layer F.Cu) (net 29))
 (segment (start 104.532168 94.92) (end 102.54 94.92) (width 0.25) (layer F.Cu) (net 29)))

